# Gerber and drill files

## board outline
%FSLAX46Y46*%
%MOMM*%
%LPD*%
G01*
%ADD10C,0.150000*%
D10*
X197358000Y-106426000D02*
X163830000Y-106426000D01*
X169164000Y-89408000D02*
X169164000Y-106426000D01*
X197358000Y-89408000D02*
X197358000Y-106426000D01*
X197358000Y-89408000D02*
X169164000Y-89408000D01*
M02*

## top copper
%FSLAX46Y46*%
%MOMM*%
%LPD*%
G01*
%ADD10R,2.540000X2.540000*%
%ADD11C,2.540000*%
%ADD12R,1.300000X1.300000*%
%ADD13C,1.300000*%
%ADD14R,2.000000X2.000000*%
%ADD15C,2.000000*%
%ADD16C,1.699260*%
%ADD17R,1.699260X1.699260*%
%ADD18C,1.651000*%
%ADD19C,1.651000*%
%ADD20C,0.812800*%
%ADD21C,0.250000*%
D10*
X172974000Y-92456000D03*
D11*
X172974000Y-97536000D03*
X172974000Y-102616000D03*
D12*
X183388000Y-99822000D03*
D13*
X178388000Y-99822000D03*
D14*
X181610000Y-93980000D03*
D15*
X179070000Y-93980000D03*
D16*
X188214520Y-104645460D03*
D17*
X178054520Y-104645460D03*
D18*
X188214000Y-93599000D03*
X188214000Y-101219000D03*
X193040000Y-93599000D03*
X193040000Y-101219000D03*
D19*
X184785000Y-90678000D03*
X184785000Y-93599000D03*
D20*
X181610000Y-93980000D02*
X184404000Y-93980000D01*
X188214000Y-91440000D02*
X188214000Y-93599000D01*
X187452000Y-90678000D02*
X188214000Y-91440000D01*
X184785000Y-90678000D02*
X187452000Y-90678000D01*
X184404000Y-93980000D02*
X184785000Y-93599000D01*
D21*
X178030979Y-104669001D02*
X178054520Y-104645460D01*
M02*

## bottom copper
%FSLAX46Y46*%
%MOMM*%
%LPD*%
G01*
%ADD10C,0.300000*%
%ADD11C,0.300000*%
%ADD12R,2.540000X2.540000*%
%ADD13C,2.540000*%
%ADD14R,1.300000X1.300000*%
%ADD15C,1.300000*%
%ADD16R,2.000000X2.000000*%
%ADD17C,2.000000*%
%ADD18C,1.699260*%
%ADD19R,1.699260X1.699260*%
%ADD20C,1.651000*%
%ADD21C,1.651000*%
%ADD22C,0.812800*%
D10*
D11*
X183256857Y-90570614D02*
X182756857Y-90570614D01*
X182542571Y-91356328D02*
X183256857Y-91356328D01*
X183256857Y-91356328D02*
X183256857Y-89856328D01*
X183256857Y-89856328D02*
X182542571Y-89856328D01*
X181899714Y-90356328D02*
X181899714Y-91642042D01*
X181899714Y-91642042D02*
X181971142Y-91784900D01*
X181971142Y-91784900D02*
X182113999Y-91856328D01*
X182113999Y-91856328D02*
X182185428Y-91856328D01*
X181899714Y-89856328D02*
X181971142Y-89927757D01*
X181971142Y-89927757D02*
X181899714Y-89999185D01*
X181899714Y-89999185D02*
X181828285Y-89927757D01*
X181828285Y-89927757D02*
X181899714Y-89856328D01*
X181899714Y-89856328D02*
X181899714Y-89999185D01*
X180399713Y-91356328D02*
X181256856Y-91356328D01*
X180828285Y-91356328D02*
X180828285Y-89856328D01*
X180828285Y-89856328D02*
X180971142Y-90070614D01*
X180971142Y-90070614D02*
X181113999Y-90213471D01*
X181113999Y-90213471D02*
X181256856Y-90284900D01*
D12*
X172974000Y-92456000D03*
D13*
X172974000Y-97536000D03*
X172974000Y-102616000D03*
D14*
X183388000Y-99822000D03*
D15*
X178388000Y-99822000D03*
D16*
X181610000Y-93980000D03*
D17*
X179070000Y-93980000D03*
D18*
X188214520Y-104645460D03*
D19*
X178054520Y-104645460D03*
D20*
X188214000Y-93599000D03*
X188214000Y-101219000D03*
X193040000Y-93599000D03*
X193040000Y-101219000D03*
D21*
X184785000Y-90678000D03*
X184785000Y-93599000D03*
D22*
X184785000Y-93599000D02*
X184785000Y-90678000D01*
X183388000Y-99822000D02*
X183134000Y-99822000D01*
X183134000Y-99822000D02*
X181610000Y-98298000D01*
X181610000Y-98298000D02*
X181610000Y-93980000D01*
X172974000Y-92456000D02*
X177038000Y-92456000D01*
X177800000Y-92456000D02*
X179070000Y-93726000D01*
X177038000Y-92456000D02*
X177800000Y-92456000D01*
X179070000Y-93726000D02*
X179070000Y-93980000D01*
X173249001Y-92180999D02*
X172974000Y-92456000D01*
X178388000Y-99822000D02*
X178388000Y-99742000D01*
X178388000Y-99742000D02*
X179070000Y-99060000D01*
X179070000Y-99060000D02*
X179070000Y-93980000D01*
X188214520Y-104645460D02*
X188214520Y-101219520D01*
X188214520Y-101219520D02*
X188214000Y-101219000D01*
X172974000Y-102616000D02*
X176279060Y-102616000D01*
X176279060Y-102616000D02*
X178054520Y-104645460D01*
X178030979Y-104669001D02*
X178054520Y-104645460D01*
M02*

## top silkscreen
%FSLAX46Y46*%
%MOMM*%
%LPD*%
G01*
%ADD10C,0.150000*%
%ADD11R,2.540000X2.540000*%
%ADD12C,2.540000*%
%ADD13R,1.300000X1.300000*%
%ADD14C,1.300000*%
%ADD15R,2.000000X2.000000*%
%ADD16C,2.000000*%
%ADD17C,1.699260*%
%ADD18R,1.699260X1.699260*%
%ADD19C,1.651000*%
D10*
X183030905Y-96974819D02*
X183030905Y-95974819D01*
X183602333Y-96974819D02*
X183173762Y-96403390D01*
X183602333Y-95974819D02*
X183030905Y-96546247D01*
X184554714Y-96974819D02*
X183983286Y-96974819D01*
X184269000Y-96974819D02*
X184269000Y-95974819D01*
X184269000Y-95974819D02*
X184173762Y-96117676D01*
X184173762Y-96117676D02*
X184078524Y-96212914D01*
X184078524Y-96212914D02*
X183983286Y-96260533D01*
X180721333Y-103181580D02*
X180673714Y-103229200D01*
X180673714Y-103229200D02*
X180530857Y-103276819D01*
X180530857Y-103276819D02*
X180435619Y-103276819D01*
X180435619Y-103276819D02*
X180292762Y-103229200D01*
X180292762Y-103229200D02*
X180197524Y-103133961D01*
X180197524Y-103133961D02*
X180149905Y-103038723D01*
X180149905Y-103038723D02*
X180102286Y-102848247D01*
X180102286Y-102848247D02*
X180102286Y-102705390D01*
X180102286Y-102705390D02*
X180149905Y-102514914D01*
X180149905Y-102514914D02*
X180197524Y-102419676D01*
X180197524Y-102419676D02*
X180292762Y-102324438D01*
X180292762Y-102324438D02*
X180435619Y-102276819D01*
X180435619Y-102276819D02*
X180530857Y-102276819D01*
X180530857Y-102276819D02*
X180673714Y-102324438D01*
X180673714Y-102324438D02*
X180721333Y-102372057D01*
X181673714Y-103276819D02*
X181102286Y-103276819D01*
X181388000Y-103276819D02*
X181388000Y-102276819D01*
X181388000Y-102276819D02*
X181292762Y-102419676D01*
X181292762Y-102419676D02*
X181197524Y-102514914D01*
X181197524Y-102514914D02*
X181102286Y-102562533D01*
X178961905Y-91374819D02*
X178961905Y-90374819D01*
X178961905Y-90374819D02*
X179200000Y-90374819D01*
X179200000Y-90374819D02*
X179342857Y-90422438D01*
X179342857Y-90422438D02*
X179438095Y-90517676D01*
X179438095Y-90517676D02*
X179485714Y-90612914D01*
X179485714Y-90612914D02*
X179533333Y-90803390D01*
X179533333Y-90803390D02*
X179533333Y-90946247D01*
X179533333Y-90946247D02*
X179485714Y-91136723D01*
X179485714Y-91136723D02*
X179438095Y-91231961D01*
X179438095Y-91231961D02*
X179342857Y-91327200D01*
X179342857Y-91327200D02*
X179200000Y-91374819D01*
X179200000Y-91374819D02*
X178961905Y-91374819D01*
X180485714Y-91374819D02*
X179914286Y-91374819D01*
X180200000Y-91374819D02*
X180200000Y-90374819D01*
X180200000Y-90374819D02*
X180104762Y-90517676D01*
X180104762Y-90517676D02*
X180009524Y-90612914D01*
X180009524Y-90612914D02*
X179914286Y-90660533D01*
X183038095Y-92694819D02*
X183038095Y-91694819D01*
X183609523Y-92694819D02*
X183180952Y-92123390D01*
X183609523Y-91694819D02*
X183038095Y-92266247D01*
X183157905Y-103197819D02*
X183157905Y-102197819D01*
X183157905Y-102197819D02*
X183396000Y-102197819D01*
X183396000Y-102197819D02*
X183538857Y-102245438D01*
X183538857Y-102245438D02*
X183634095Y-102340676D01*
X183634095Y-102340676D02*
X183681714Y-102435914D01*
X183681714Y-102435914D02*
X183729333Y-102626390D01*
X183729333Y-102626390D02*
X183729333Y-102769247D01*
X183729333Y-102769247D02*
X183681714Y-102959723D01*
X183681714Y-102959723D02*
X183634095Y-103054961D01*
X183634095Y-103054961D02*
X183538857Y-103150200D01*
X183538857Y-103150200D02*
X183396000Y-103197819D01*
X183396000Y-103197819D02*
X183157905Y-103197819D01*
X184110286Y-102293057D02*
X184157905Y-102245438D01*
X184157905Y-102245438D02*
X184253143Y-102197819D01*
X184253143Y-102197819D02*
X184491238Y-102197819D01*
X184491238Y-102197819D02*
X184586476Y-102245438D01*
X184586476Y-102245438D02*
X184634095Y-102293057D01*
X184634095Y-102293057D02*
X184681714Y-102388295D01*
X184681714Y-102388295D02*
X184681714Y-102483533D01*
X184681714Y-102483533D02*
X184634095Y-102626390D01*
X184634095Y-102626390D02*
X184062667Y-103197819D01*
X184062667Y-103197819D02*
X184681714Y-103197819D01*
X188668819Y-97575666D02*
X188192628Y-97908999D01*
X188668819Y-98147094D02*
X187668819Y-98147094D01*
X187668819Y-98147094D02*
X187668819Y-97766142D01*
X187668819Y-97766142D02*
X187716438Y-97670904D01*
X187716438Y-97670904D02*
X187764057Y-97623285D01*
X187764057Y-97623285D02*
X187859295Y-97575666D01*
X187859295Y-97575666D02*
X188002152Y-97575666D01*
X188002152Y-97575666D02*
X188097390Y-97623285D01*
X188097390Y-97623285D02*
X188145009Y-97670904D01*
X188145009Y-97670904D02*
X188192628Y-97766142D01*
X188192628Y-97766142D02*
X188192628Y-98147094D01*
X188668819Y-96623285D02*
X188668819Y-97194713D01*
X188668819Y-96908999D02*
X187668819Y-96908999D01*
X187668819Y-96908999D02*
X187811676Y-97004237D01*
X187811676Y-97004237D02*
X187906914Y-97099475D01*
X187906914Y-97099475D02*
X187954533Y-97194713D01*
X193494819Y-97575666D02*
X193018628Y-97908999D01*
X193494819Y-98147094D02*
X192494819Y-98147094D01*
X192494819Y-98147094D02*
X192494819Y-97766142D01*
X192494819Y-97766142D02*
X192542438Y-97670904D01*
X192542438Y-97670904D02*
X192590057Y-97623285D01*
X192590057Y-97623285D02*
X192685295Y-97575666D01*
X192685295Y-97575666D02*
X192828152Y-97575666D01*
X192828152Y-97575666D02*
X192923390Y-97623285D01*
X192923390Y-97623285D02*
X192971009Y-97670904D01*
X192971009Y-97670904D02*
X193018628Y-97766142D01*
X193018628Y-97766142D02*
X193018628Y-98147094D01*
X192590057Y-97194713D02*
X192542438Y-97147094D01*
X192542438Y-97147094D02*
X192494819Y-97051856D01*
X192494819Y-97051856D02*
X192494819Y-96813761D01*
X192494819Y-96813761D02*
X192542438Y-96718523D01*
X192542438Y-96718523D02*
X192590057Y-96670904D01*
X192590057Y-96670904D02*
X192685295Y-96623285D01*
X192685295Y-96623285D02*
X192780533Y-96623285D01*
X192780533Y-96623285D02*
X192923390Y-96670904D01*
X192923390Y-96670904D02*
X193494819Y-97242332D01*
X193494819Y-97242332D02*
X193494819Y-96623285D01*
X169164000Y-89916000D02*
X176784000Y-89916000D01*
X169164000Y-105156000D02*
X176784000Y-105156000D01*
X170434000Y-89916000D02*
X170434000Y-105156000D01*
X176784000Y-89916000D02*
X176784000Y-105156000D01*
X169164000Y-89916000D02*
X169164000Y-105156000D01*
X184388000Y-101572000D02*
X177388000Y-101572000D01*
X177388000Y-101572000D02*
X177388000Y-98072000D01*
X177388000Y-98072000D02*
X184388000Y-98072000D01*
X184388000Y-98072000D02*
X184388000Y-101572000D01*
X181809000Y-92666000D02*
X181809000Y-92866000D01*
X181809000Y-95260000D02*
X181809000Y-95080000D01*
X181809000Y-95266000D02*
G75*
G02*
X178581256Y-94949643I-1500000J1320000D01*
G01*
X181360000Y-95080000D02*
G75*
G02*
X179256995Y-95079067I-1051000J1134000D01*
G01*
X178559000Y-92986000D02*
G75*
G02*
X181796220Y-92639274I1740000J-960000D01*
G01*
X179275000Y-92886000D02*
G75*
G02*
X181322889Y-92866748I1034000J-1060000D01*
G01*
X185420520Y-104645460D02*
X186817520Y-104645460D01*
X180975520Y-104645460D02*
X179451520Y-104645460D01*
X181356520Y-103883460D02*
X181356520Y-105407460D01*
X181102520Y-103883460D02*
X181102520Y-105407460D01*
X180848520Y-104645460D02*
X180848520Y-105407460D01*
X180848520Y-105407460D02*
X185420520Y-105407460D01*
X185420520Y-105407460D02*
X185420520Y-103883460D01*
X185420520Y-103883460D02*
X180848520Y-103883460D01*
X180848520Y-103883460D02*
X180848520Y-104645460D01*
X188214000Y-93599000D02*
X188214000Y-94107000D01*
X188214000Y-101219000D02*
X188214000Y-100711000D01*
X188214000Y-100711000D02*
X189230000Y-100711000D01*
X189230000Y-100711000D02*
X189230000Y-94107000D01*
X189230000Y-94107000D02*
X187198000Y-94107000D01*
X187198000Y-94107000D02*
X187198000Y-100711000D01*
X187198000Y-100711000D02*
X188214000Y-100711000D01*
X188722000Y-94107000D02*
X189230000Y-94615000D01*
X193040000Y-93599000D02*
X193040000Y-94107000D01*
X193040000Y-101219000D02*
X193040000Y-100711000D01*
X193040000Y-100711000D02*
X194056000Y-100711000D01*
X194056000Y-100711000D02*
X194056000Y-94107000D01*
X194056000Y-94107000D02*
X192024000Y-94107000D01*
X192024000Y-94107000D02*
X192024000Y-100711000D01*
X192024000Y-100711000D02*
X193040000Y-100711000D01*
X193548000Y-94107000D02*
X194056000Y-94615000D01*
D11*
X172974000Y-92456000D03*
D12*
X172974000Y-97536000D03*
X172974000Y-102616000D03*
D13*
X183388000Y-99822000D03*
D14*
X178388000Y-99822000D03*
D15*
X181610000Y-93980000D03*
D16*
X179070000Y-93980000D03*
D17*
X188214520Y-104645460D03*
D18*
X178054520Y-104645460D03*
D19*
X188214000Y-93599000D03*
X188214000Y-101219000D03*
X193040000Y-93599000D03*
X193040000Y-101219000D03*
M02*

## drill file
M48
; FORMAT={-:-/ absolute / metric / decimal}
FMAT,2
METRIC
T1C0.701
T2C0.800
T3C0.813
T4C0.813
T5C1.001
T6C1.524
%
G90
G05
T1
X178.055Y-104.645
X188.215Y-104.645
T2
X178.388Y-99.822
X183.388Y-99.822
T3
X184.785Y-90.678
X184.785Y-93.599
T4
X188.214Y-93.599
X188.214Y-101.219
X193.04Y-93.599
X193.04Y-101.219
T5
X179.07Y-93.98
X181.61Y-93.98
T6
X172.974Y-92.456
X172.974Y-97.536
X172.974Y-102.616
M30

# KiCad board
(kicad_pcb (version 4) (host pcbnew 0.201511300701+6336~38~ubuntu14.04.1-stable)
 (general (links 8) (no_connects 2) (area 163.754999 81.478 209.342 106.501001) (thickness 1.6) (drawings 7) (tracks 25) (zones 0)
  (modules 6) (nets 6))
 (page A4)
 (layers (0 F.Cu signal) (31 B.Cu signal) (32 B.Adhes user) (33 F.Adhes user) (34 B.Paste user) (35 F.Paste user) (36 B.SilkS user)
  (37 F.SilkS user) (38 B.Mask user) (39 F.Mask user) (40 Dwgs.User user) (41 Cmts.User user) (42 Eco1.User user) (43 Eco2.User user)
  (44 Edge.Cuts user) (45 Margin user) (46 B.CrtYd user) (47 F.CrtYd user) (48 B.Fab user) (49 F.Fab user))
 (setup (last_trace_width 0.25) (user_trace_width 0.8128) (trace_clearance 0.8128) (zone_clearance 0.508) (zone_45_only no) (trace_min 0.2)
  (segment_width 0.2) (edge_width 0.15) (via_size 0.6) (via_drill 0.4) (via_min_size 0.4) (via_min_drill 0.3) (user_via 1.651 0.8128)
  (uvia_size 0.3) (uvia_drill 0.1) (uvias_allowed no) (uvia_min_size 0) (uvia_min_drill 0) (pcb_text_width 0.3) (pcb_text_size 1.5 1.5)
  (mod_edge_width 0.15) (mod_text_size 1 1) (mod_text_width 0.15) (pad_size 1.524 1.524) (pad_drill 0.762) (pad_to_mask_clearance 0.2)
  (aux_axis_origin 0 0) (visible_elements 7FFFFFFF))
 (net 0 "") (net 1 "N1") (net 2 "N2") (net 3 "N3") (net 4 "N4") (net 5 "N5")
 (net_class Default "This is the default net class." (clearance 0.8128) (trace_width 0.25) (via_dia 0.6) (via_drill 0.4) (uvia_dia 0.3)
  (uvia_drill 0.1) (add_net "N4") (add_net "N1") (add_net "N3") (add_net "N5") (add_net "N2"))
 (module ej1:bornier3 (layer F.Cu) (at 172.974 97.536 270)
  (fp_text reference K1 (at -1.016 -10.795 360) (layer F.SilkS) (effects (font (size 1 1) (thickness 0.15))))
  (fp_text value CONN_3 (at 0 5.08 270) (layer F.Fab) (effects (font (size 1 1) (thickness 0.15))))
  (fp_line (start -7.62 3.81) (end -7.62 -3.81) (layer F.SilkS) (width 0.15))
  (fp_line (start 7.62 3.81) (end 7.62 -3.81) (layer F.SilkS) (width 0.15))
  (fp_line (start -7.62 2.54) (end 7.62 2.54) (layer F.SilkS) (width 0.15))
  (fp_line (start -7.62 -3.81) (end 7.62 -3.81) (layer F.SilkS) (width 0.15))
  (fp_line (start -7.62 3.81) (end 7.62 3.81) (layer F.SilkS) (width 0.15))
  (pad 1 thru_hole rect (at -5.08 0 270) (size 2.54 2.54) (drill 1.524) (layers *.Cu *.Mask F.SilkS) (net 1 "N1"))
  (pad 2 thru_hole circle (at 0 0 270) (size 2.54 2.54) (drill 1.524) (layers *.Cu *.Mask F.SilkS) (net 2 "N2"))
  (pad 3 thru_hole circle (at 5.08 0 270) (size 2.54 2.54) (drill 1.524) (layers *.Cu *.Mask F.SilkS) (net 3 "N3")))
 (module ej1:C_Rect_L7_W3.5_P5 (layer F.Cu) (at 183.388 99.822 180)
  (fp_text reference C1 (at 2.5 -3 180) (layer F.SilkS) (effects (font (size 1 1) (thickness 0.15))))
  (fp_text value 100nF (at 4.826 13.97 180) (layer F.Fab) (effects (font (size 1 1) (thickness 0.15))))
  (fp_line (start -1 -1.75) (end 6 -1.75) (layer F.SilkS) (width 0.15))
  (fp_line (start 6 -1.75) (end 6 1.75) (layer F.SilkS) (width 0.15))
  (fp_line (start 6 1.75) (end -1 1.75) (layer F.SilkS) (width 0.15))
  (fp_line (start -1 1.75) (end -1 -1.75) (layer F.SilkS) (width 0.15))
  (pad 1 thru_hole rect (at 0 0 180) (size 1.3 1.3) (drill 0.8) (layers *.Cu *.Mask F.SilkS) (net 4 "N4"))
  (pad 2 thru_hole circle (at 5 0 180) (size 1.3 1.3) (drill 0.8) (layers *.Cu *.Mask F.SilkS) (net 1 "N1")))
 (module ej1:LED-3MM (layer F.Cu) (at 181.61 93.98 180)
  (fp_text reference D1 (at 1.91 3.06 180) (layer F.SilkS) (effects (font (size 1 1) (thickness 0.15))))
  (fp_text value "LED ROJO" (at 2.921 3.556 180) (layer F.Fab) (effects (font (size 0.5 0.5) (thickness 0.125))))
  (fp_line (start -0.199 1.314) (end -0.199 1.114) (layer F.SilkS) (width 0.15))
  (fp_line (start -0.199 -1.28) (end -0.199 -1.1) (layer F.SilkS) (width 0.15))
  (fp_arc (start 1.301 0.034) (end -0.199 -1.286) (angle 108.5) (layer F.SilkS) (width 0.15))
  (fp_arc (start 1.301 0.034) (end 0.25 -1.1) (angle 85.7) (layer F.SilkS) (width 0.15))
  (fp_arc (start 1.311 0.034) (end 3.051 0.994) (angle 110) (layer F.SilkS) (width 0.15))
  (fp_arc (start 1.301 0.034) (end 2.335 1.094) (angle 87.5) (layer F.SilkS) (width 0.15))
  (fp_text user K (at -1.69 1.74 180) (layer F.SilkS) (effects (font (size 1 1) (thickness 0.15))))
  (pad 1 thru_hole rect (at 0 0 270) (size 2 2) (drill 1.00076) (layers *.Cu *.Mask F.SilkS) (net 4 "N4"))
  (pad 2 thru_hole circle (at 2.54 0 180) (size 2 2) (drill 1.00076) (layers *.Cu *.Mask F.SilkS) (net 1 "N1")))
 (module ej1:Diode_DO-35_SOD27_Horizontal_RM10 (layer F.Cu) (at 178.054 104.648)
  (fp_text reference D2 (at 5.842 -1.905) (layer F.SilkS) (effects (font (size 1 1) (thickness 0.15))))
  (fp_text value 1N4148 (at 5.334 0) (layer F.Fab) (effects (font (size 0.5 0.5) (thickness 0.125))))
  (fp_line (start 7.36652 -0.00254) (end 8.76352 -0.00254) (layer F.SilkS) (width 0.15))
  (fp_line (start 2.92152 -0.00254) (end 1.39752 -0.00254) (layer F.SilkS) (width 0.15))
  (fp_line (start 3.30252 -0.76454) (end 3.30252 0.75946) (layer F.SilkS) (width 0.15))
  (fp_line (start 3.04852 -0.76454) (end 3.04852 0.75946) (layer F.SilkS) (width 0.15))
  (fp_line (start 2.79452 -0.00254) (end 2.79452 0.75946) (layer F.SilkS) (width 0.15))
  (fp_line (start 2.79452 0.75946) (end 7.36652 0.75946) (layer F.SilkS) (width 0.15))
  (fp_line (start 7.36652 0.75946) (end 7.36652 -0.76454) (layer F.SilkS) (width 0.15))
  (fp_line (start 7.36652 -0.76454) (end 2.79452 -0.76454) (layer F.SilkS) (width 0.15))
  (fp_line (start 2.79452 -0.76454) (end 2.79452 -0.00254) (layer F.SilkS) (width 0.15))
  (pad 2 thru_hole circle (at 10.16052 -0.00254 180) (size 1.69926 1.69926) (drill 0.70104) (layers *.Cu *.Mask F.SilkS) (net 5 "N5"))
  (pad 1 thru_hole rect (at 0.00052 -0.00254 180) (size 1.69926 1.69926) (drill 0.70104) (layers *.Cu *.Mask F.SilkS) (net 3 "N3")))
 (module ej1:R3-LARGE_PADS (layer F.Cu) (at 188.214 97.409 270)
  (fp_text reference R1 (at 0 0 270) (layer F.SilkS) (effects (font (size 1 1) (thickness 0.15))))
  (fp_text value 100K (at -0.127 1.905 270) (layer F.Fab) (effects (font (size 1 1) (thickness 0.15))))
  (fp_line (start -3.81 0) (end -3.302 0) (layer F.SilkS) (width 0.15))
  (fp_line (start 3.81 0) (end 3.302 0) (layer F.SilkS) (width 0.15))
  (fp_line (start 3.302 0) (end 3.302 -1.016) (layer F.SilkS) (width 0.15))
  (fp_line (start 3.302 -1.016) (end -3.302 -1.016) (layer F.SilkS) (width 0.15))
  (fp_line (start -3.302 -1.016) (end -3.302 1.016) (layer F.SilkS) (width 0.15))
  (fp_line (start -3.302 1.016) (end 3.302 1.016) (layer F.SilkS) (width 0.15))
  (fp_line (start 3.302 1.016) (end 3.302 0) (layer F.SilkS) (width 0.15))
  (fp_line (start -3.302 -0.508) (end -2.794 -1.016) (layer F.SilkS) (width 0.15))
  (pad 1 thru_hole circle (at -3.81 0 270) (size 1.651 1.651) (drill 0.8128) (layers *.Cu *.Mask F.SilkS) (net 4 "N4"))
  (pad 2 thru_hole circle (at 3.81 0 270) (size 1.651 1.651) (drill 0.8128) (layers *.Cu *.Mask F.SilkS) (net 5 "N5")))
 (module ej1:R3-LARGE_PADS (layer F.Cu) (at 193.04 97.409 270)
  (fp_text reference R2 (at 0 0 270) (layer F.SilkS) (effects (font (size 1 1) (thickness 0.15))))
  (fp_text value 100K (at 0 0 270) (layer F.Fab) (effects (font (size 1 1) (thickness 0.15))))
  (fp_line (start -3.81 0) (end -3.302 0) (layer F.SilkS) (width 0.15))
  (fp_line (start 3.81 0) (end 3.302 0) (layer F.SilkS) (width 0.15))
  (fp_line (start 3.302 0) (end 3.302 -1.016) (layer F.SilkS) (width 0.15))
  (fp_line (start 3.302 -1.016) (end -3.302 -1.016) (layer F.SilkS) (width 0.15))
  (fp_line (start -3.302 -1.016) (end -3.302 1.016) (layer F.SilkS) (width 0.15))
  (fp_line (start -3.302 1.016) (end 3.302 1.016) (layer F.SilkS) (width 0.15))
  (fp_line (start 3.302 1.016) (end 3.302 0) (layer F.SilkS) (width 0.15))
  (fp_line (start -3.302 -0.508) (end -2.794 -1.016) (layer F.SilkS) (width 0.15))
  (pad 1 thru_hole circle (at -3.81 0 270) (size 1.651 1.651) (drill 0.8128) (layers *.Cu *.Mask F.SilkS) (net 4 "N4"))
  (pad 2 thru_hole circle (at 3.81 0 270) (size 1.651 1.651) (drill 0.8128) (layers *.Cu *.Mask F.SilkS) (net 5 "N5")))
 (gr_line (start 197.358 106.426) (end 163.83 106.426) (angle 90) (layer Edge.Cuts) (width 0.15))
 (gr_line (start 169.164 89.408) (end 169.164 106.426) (angle 90) (layer Edge.Cuts) (width 0.15))
 (gr_line (start 197.358 89.408) (end 197.358 106.426) (angle 90) (layer Edge.Cuts) (width 0.15))
 (gr_line (start 197.358 89.408) (end 169.164 89.408) (angle 90) (layer Edge.Cuts) (width 0.15))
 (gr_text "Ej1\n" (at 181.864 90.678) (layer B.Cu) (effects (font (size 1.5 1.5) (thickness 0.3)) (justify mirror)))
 (segment (start 181.61 93.98) (end 184.404 93.98) (width 0.8128) (layer F.Cu) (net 4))
 (segment (start 188.214 91.44) (end 188.214 93.599) (width 0.8128) (layer F.Cu) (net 4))
 (segment (start 187.452 90.678) (end 188.214 91.44) (width 0.8128) (layer F.Cu) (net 4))
 (segment (start 184.785 90.678) (end 187.452 90.678) (width 0.8128) (layer F.Cu) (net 4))
 (via (at 184.785 90.678) (size 1.651) (drill 0.8128) (layers F.Cu B.Cu) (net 4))
 (segment (start 184.785 93.599) (end 184.785 90.678) (width 0.8128) (layer B.Cu) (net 4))
 (via (at 184.785 93.599) (size 1.651) (drill 0.8128) (layers F.Cu B.Cu) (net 4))
 (segment (start 184.404 93.98) (end 184.785 93.599) (width 0.8128) (layer F.Cu) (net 4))
 (segment (start 183.388 99.822) (end 183.134 99.822) (width 0.8128) (layer B.Cu) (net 4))
 (segment (start 183.134 99.822) (end 181.61 98.298) (width 0.8128) (layer B.Cu) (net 4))
 (segment (start 181.61 98.298) (end 181.61 93.98) (width 0.8128) (layer B.Cu) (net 4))
 (segment (start 172.974 92.456) (end 177.038 92.456) (width 0.8128) (layer B.Cu) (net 1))
 (segment (start 177.8 92.456) (end 179.07 93.726) (width 0.8128) (layer B.Cu) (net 1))
 (segment (start 177.038 92.456) (end 177.8 92.456) (width 0.8128) (layer B.Cu) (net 1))
 (segment (start 179.07 93.726) (end 179.07 93.98) (width 0.8128) (layer B.Cu) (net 1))
 (segment (start 173.249001 92.180999) (end 172.974 92.456) (width 0.8128) (layer B.Cu) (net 1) (status 30))
 (segment (start 178.388 99.822) (end 178.388 99.742) (width 0.8128) (layer B.Cu) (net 1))
 (segment (start 178.388 99.742) (end 179.07 99.06) (width 0.8128) (layer B.Cu) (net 1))
 (segment (start 179.07 99.06) (end 179.07 93.98) (width 0.8128) (layer B.Cu) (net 1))
 (segment (start 188.21452 104.64546) (end 188.21452 101.21952) (width 0.8128) (layer B.Cu) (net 5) (status 10))
 (segment (start 188.21452 101.21952) (end 188.214 101.219) (width 0.8128) (layer B.Cu) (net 5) (status 30))
 (segment (start 172.974 102.616) (end 176.27906 102.616) (width 0.8128) (layer B.Cu) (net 3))
 (segment (start 176.27906 102.616) (end 178.05452 104.64546) (width 0.8128) (layer B.Cu) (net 3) (status 20))
 (segment (start 178.030979 104.669001) (end 178.05452 104.64546) (width 0.8128) (layer B.Cu) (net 3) (status 30))
 (segment (start 178.030979 104.669001) (end 178.05452 104.64546) (width 0.25) (layer F.Cu) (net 3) (status 30)))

